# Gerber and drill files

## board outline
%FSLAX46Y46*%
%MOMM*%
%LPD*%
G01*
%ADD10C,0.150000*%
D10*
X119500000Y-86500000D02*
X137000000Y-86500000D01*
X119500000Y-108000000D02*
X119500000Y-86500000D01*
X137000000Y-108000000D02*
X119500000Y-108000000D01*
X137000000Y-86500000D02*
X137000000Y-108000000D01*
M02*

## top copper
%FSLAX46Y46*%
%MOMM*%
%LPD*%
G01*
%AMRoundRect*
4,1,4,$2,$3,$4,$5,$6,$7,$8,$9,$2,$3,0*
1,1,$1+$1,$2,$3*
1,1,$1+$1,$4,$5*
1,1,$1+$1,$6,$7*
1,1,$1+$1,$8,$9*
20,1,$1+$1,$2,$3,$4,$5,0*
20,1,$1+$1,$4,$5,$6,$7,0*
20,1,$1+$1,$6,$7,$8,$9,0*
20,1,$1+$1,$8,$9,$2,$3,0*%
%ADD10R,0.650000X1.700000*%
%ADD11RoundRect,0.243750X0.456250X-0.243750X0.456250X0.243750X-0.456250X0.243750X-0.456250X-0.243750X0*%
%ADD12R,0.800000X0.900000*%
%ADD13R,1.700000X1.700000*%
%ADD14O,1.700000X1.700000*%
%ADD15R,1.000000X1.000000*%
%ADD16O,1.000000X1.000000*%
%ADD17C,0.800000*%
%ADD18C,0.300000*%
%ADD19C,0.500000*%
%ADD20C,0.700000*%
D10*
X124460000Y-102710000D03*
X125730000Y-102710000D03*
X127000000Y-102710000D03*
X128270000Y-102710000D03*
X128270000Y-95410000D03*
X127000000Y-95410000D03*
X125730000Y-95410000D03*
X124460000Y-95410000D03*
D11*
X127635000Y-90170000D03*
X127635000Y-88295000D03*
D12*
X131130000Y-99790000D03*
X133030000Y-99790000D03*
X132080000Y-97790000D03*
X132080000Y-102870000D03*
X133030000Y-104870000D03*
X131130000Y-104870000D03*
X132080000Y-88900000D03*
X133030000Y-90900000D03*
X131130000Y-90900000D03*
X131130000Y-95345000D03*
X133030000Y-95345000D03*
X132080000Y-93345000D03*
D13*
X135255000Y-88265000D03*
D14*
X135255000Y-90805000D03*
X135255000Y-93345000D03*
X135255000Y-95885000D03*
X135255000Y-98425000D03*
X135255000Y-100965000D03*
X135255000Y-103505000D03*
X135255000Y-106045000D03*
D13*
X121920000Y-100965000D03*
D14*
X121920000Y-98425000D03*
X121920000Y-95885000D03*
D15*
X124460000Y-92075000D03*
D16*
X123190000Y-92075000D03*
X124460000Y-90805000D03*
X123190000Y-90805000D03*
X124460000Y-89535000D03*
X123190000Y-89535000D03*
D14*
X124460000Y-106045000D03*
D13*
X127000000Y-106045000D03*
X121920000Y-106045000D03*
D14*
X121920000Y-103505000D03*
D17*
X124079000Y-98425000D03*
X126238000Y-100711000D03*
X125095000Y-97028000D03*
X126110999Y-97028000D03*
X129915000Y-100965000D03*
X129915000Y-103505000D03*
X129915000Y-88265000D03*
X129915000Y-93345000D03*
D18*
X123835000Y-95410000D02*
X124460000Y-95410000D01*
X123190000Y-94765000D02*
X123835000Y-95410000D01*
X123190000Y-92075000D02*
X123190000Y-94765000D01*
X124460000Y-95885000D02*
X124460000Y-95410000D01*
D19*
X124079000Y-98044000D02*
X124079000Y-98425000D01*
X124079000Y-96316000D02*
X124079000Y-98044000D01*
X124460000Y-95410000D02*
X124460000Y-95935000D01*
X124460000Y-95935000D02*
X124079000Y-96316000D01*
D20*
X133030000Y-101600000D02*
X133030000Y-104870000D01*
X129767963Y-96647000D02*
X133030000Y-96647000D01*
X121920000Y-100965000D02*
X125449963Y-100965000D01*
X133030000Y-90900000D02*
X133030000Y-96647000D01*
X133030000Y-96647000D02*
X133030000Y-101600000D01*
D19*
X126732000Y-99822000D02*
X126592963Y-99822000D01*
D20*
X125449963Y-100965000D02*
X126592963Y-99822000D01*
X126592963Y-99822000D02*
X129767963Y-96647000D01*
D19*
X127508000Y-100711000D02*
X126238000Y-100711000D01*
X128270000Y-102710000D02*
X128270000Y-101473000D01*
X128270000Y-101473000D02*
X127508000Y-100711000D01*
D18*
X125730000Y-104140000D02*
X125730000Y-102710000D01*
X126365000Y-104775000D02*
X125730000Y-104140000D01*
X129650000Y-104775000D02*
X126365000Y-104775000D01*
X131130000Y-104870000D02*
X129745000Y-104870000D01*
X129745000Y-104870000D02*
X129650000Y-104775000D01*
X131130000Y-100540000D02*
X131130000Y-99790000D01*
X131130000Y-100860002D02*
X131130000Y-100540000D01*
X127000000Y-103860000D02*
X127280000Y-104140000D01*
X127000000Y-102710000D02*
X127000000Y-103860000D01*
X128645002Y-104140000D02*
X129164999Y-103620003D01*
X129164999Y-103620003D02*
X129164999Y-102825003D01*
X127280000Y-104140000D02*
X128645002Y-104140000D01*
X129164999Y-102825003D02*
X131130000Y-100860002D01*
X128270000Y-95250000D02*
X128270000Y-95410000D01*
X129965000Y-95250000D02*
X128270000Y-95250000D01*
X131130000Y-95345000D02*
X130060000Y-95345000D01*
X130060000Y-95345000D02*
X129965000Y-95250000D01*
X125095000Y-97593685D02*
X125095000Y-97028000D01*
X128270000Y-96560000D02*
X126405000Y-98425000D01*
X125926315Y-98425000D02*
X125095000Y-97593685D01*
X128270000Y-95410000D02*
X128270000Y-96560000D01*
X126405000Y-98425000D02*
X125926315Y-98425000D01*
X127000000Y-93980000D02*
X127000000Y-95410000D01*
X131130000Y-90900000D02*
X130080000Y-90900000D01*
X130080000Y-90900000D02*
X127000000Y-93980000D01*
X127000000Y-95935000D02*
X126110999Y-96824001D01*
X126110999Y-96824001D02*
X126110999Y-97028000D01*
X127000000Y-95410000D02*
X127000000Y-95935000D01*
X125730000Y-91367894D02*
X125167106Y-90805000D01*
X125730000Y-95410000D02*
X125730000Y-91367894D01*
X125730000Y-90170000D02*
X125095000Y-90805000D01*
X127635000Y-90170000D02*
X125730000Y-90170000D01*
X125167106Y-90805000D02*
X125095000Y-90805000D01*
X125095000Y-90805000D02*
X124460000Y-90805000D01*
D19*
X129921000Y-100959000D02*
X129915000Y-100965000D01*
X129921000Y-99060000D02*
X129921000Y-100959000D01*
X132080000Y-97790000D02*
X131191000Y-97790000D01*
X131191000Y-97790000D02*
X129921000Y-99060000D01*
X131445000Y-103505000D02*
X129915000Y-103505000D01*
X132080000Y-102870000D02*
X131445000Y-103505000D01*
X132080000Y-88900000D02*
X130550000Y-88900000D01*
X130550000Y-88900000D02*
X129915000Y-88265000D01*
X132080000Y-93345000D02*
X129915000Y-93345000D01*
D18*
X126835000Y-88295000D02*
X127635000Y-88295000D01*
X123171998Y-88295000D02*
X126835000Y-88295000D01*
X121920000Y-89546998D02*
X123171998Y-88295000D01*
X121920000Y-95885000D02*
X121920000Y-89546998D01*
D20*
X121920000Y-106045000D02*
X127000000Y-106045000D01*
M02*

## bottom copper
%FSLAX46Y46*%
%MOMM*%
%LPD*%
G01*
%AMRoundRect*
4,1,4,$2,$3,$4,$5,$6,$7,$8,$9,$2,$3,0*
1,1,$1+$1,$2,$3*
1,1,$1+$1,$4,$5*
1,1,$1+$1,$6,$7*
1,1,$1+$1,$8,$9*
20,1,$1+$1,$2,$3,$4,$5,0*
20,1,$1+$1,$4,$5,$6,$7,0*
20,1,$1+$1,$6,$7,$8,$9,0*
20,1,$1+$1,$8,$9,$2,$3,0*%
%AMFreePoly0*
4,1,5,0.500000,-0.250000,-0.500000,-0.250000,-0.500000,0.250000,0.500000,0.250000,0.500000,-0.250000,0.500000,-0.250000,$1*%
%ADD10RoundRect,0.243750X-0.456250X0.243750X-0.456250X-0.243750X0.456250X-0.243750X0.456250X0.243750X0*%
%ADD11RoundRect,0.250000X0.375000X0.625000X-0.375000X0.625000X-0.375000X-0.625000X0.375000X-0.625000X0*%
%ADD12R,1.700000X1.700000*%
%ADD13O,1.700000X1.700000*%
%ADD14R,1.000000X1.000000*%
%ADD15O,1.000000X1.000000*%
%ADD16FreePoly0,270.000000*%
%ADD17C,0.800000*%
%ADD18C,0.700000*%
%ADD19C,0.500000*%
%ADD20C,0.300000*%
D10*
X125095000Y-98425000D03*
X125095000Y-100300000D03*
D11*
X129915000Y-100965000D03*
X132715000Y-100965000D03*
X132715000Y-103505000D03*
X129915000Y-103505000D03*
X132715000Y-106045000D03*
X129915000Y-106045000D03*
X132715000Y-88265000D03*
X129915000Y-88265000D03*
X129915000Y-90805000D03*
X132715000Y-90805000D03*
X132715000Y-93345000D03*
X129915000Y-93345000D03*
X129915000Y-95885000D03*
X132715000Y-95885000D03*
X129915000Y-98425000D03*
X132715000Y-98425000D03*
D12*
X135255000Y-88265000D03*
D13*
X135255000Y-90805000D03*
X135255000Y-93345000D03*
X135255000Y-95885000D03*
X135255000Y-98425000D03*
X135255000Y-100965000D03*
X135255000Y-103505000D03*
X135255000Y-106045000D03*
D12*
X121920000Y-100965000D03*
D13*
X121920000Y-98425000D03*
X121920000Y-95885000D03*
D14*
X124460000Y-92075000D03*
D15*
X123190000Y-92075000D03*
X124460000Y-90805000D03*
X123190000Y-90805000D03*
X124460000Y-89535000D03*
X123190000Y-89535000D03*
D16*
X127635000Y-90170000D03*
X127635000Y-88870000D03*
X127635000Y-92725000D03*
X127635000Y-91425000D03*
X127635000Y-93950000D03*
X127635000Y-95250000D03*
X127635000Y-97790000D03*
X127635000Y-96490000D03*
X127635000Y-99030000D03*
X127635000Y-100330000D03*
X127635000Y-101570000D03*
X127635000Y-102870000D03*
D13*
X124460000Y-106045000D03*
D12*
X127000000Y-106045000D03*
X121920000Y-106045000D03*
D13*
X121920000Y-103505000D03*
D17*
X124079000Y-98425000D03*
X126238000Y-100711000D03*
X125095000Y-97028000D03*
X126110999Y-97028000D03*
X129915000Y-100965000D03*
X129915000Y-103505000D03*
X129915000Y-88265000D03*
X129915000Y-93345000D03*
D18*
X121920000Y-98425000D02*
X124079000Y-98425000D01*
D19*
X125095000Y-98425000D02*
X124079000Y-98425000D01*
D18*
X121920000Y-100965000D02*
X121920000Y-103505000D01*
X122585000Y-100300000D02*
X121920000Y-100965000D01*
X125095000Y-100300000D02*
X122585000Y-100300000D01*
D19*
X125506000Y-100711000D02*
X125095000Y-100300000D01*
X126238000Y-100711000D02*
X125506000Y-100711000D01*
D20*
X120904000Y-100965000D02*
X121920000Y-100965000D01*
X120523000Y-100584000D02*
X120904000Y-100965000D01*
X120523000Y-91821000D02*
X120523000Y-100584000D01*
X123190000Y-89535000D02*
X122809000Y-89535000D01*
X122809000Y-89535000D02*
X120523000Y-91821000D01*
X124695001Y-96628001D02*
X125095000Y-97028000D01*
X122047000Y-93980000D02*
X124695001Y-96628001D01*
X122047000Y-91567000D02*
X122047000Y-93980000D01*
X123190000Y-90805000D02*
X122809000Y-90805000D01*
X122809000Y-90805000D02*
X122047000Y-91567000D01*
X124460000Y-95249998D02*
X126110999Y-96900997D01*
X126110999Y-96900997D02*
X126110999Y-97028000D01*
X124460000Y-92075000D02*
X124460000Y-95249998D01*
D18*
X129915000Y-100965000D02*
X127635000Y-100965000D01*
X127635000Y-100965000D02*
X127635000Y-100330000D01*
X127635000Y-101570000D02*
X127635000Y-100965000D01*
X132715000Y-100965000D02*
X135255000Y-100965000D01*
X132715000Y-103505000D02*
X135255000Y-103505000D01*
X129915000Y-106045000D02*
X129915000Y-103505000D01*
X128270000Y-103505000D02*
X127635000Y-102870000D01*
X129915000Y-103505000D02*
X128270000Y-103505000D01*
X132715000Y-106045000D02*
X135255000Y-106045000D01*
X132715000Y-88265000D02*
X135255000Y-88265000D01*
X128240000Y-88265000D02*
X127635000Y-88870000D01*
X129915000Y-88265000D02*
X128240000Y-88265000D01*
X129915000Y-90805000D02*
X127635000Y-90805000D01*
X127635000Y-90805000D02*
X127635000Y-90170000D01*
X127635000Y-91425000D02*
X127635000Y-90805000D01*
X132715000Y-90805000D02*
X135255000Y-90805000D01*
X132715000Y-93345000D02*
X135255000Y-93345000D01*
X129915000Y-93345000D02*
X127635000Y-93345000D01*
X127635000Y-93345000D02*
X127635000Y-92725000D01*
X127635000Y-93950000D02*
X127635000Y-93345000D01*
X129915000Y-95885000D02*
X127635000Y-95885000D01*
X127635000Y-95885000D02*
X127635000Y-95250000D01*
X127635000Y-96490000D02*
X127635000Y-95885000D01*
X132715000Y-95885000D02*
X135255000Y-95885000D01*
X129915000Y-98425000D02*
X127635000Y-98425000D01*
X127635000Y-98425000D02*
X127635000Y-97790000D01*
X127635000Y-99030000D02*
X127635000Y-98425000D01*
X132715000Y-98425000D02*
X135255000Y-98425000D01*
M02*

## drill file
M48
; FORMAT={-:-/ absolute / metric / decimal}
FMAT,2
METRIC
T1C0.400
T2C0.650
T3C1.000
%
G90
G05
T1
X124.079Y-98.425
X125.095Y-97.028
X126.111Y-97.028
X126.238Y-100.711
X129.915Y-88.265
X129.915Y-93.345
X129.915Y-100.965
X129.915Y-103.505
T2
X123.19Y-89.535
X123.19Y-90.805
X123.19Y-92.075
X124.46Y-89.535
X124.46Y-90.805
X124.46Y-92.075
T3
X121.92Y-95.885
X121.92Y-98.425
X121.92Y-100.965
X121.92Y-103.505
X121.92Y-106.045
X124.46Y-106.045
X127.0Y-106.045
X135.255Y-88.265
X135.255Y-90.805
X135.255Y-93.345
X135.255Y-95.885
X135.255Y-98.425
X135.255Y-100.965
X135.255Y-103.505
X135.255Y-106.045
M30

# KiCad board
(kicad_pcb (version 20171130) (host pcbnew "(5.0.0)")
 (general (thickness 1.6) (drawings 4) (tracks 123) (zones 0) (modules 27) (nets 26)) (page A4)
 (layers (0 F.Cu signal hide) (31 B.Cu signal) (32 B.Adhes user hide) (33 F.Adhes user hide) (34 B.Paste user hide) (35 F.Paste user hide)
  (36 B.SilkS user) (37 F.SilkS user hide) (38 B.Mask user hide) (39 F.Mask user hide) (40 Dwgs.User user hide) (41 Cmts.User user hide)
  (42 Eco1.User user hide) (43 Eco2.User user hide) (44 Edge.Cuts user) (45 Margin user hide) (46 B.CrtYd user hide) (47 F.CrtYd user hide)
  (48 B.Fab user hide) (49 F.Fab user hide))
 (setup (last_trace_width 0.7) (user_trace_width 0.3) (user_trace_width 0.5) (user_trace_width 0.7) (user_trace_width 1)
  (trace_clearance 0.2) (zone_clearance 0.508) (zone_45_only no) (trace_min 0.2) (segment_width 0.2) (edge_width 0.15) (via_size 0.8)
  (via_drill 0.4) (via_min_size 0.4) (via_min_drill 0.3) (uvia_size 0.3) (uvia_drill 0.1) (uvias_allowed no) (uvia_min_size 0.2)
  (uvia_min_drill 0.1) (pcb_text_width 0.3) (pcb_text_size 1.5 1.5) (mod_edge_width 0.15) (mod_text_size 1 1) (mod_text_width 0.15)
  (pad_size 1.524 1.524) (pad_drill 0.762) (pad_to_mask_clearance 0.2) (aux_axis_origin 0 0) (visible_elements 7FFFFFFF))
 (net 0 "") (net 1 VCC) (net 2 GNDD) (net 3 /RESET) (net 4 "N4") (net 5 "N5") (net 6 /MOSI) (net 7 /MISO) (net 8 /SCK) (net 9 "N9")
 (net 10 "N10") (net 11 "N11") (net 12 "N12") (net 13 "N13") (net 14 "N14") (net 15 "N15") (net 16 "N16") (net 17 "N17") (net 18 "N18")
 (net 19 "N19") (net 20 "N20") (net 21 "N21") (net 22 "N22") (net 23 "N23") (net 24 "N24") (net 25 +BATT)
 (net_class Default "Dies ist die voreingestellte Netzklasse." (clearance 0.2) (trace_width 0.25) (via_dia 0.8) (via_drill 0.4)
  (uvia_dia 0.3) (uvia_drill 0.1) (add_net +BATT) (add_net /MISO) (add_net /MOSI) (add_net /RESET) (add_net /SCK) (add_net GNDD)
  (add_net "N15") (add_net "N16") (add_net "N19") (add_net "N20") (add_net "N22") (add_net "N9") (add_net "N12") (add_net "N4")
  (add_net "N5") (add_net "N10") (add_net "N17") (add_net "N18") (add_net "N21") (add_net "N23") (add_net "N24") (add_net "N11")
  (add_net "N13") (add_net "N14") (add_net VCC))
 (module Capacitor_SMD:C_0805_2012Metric (layer B.Cu) (at 125.095 99.3625 270)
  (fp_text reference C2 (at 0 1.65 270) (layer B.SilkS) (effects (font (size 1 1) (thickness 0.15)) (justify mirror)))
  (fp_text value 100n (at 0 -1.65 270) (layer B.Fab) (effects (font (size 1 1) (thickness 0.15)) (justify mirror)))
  (pad 1 smd roundrect (at -0.9375 0 270) (size 0.975 1.4) (layers B.Cu B.Paste B.Mask) (roundrect_rratio 0.25) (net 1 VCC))
  (pad 2 smd roundrect (at 0.9375 0 270) (size 0.975 1.4) (layers B.Cu B.Paste B.Mask) (roundrect_rratio 0.25) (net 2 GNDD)))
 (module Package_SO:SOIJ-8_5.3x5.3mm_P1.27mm (layer F.Cu) (at 126.365 99.06 90)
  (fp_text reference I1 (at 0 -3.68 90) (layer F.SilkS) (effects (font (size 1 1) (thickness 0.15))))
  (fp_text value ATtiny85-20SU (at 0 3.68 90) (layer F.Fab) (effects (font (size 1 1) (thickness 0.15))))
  (pad 1 smd rect (at -3.65 -1.905 90) (size 1.7 0.65) (layers F.Cu F.Paste F.Mask) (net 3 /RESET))
  (pad 2 smd rect (at -3.65 -0.635 90) (size 1.7 0.65) (layers F.Cu F.Paste F.Mask) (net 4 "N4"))
  (pad 3 smd rect (at -3.65 0.635 90) (size 1.7 0.65) (layers F.Cu F.Paste F.Mask) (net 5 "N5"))
  (pad 4 smd rect (at -3.65 1.905 90) (size 1.7 0.65) (layers F.Cu F.Paste F.Mask) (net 2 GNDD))
  (pad 5 smd rect (at 3.65 1.905 90) (size 1.7 0.65) (layers F.Cu F.Paste F.Mask) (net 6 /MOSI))
  (pad 6 smd rect (at 3.65 0.635 90) (size 1.7 0.65) (layers F.Cu F.Paste F.Mask) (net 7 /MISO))
  (pad 7 smd rect (at 3.65 -0.635 90) (size 1.7 0.65) (layers F.Cu F.Paste F.Mask) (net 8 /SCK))
  (pad 8 smd rect (at 3.65 -1.905 90) (size 1.7 0.65) (layers F.Cu F.Paste F.Mask) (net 1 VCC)))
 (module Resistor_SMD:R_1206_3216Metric (layer B.Cu) (at 131.315 100.965 180)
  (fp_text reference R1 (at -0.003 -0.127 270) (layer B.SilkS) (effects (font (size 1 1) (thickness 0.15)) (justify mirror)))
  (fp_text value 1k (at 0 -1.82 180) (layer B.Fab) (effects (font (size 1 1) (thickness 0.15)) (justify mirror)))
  (pad 2 smd roundrect (at 1.4 0 180) (size 1.25 1.75) (layers B.Cu B.Paste B.Mask) (roundrect_rratio 0.2) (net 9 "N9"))
  (pad 1 smd roundrect (at -1.4 0 180) (size 1.25 1.75) (layers B.Cu B.Paste B.Mask) (roundrect_rratio 0.2) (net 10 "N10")))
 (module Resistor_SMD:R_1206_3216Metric (layer B.Cu) (at 131.315 103.505 180)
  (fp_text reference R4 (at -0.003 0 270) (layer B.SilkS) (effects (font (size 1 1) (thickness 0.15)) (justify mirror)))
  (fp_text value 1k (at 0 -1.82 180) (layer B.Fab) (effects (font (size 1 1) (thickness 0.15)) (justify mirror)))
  (pad 1 smd roundrect (at -1.4 0 180) (size 1.25 1.75) (layers B.Cu B.Paste B.Mask) (roundrect_rratio 0.2) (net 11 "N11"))
  (pad 2 smd roundrect (at 1.4 0 180) (size 1.25 1.75) (layers B.Cu B.Paste B.Mask) (roundrect_rratio 0.2) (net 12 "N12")))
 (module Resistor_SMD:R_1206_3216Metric (layer B.Cu) (at 131.315 106.045 180)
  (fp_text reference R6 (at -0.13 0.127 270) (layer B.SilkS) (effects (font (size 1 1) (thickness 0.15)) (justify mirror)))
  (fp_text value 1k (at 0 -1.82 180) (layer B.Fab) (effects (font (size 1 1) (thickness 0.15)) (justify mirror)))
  (pad 1 smd roundrect (at -1.4 0 180) (size 1.25 1.75) (layers B.Cu B.Paste B.Mask) (roundrect_rratio 0.2) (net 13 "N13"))
  (pad 2 smd roundrect (at 1.4 0 180) (size 1.25 1.75) (layers B.Cu B.Paste B.Mask) (roundrect_rratio 0.2) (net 12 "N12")))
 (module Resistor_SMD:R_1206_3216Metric (layer B.Cu) (at 131.315 88.265 180)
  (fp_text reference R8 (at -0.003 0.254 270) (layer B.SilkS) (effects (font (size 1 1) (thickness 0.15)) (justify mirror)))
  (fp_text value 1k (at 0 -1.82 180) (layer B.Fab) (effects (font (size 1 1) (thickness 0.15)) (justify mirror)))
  (pad 1 smd roundrect (at -1.4 0 180) (size 1.25 1.75) (layers B.Cu B.Paste B.Mask) (roundrect_rratio 0.2) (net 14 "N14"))
  (pad 2 smd roundrect (at 1.4 0 180) (size 1.25 1.75) (layers B.Cu B.Paste B.Mask) (roundrect_rratio 0.2) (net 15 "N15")))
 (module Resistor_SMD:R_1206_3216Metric (layer B.Cu) (at 131.315 90.805 180)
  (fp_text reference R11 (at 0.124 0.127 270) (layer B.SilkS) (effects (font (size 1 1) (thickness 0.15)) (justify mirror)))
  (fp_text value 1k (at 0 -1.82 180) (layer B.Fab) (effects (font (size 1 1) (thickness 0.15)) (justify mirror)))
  (pad 2 smd roundrect (at 1.4 0 180) (size 1.25 1.75) (layers B.Cu B.Paste B.Mask) (roundrect_rratio 0.2) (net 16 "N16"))
  (pad 1 smd roundrect (at -1.4 0 180) (size 1.25 1.75) (layers B.Cu B.Paste B.Mask) (roundrect_rratio 0.2) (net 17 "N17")))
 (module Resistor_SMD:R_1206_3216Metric (layer B.Cu) (at 131.315 93.345 180)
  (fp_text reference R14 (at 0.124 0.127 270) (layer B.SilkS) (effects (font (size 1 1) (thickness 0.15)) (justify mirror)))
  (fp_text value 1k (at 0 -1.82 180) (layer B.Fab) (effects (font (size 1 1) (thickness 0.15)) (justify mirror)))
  (pad 1 smd roundrect (at -1.4 0 180) (size 1.25 1.75) (layers B.Cu B.Paste B.Mask) (roundrect_rratio 0.2) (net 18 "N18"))
  (pad 2 smd roundrect (at 1.4 0 180) (size 1.25 1.75) (layers B.Cu B.Paste B.Mask) (roundrect_rratio 0.2) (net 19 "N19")))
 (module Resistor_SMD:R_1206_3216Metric (layer B.Cu) (at 131.315 95.885 180)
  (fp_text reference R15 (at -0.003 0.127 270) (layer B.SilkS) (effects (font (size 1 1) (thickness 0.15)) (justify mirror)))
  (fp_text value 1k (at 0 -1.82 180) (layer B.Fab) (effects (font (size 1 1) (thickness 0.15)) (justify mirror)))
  (pad 2 smd roundrect (at 1.4 0 180) (size 1.25 1.75) (layers B.Cu B.Paste B.Mask) (roundrect_rratio 0.2) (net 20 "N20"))
  (pad 1 smd roundrect (at -1.4 0 180) (size 1.25 1.75) (layers B.Cu B.Paste B.Mask) (roundrect_rratio 0.2) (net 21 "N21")))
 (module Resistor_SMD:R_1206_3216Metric (layer B.Cu) (at 131.315 98.425 180)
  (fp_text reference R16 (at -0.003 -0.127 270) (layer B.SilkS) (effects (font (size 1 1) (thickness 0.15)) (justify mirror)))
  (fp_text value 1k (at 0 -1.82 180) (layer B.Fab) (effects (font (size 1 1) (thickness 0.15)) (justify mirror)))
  (pad 2 smd roundrect (at 1.4 0 180) (size 1.25 1.75) (layers B.Cu B.Paste B.Mask) (roundrect_rratio 0.2) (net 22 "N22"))
  (pad 1 smd roundrect (at -1.4 0 180) (size 1.25 1.75) (layers B.Cu B.Paste B.Mask) (roundrect_rratio 0.2) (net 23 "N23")))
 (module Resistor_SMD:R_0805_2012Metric (layer F.Cu) (at 127.635 89.2325 90)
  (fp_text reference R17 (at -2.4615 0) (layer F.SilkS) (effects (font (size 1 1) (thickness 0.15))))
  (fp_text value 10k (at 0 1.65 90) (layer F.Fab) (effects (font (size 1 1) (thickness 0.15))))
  (pad 1 smd roundrect (at -0.9375 0 90) (size 0.975 1.4) (layers F.Cu F.Paste F.Mask) (roundrect_rratio 0.25) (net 8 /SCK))
  (pad 2 smd roundrect (at 0.9375 0 90) (size 0.975 1.4) (layers F.Cu F.Paste F.Mask) (roundrect_rratio 0.25) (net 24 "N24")))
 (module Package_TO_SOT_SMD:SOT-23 (layer F.Cu) (at 132.08 98.79 90)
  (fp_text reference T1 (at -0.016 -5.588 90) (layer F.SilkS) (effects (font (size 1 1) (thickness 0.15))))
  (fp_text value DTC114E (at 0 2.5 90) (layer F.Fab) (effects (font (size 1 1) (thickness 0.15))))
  (pad 1 smd rect (at -1 -0.95 90) (size 0.9 0.8) (layers F.Cu F.Paste F.Mask) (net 5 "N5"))
  (pad 2 smd rect (at -1 0.95 90) (size 0.9 0.8) (layers F.Cu F.Paste F.Mask) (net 2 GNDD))
  (pad 3 smd rect (at 1 0 90) (size 0.9 0.8) (layers F.Cu F.Paste F.Mask) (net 9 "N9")))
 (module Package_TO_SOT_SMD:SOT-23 (layer F.Cu) (at 132.08 103.87 90)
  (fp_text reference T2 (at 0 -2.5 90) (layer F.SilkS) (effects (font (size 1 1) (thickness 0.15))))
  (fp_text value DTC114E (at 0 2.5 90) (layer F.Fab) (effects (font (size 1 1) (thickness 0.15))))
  (pad 3 smd rect (at 1 0 90) (size 0.9 0.8) (layers F.Cu F.Paste F.Mask) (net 12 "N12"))
  (pad 2 smd rect (at -1 0.95 90) (size 0.9 0.8) (layers F.Cu F.Paste F.Mask) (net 2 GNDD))
  (pad 1 smd rect (at -1 -0.95 90) (size 0.9 0.8) (layers F.Cu F.Paste F.Mask) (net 4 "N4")))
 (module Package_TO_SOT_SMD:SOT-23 (layer F.Cu) (at 132.08 89.9 90)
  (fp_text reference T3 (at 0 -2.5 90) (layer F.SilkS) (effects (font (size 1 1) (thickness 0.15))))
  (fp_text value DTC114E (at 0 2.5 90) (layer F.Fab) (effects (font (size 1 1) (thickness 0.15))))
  (pad 3 smd rect (at 1 0 90) (size 0.9 0.8) (layers F.Cu F.Paste F.Mask) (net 15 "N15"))
  (pad 2 smd rect (at -1 0.95 90) (size 0.9 0.8) (layers F.Cu F.Paste F.Mask) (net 2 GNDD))
  (pad 1 smd rect (at -1 -0.95 90) (size 0.9 0.8) (layers F.Cu F.Paste F.Mask) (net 7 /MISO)))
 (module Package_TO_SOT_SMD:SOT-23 (layer F.Cu) (at 132.08 94.345 90)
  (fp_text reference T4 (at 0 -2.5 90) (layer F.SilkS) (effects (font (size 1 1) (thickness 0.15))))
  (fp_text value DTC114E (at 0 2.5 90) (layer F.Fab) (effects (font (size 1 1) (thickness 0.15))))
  (pad 1 smd rect (at -1 -0.95 90) (size 0.9 0.8) (layers F.Cu F.Paste F.Mask) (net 6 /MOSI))
  (pad 2 smd rect (at -1 0.95 90) (size 0.9 0.8) (layers F.Cu F.Paste F.Mask) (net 2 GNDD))
  (pad 3 smd rect (at 1 0 90) (size 0.9 0.8) (layers F.Cu F.Paste F.Mask) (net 19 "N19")))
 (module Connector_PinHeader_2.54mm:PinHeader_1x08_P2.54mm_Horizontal (layer F.Cu) (at 135.255 88.265)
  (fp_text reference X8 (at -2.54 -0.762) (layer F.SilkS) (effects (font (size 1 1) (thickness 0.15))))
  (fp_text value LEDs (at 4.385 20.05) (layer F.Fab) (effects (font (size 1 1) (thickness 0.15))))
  (pad 1 thru_hole rect (at 0 0) (size 1.7 1.7) (drill 1) (layers *.Cu *.Mask) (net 14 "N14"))
  (pad 2 thru_hole oval (at 0 2.54) (size 1.7 1.7) (drill 1) (layers *.Cu *.Mask) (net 17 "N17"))
  (pad 3 thru_hole oval (at 0 5.08) (size 1.7 1.7) (drill 1) (layers *.Cu *.Mask) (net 18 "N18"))
  (pad 4 thru_hole oval (at 0 7.62) (size 1.7 1.7) (drill 1) (layers *.Cu *.Mask) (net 21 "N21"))
  (pad 5 thru_hole oval (at 0 10.16) (size 1.7 1.7) (drill 1) (layers *.Cu *.Mask) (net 23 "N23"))
  (pad 6 thru_hole oval (at 0 12.7) (size 1.7 1.7) (drill 1) (layers *.Cu *.Mask) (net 10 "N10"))
  (pad 7 thru_hole oval (at 0 15.24) (size 1.7 1.7) (drill 1) (layers *.Cu *.Mask) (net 11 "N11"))
  (pad 8 thru_hole oval (at 0 17.78) (size 1.7 1.7) (drill 1) (layers *.Cu *.Mask) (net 13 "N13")))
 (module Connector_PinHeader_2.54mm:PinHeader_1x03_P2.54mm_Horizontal (layer F.Cu) (at 121.92 100.965 180)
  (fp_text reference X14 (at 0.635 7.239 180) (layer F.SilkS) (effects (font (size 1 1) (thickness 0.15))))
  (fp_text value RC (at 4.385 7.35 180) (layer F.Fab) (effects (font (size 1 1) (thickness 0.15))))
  (pad 1 thru_hole rect (at 0 0 180) (size 1.7 1.7) (drill 1) (layers *.Cu *.Mask) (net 2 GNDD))
  (pad 2 thru_hole oval (at 0 2.54 180) (size 1.7 1.7) (drill 1) (layers *.Cu *.Mask) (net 1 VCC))
  (pad 3 thru_hole oval (at 0 5.08 180) (size 1.7 1.7) (drill 1) (layers *.Cu *.Mask) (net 24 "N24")))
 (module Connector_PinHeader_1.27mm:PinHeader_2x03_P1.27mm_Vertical (layer F.Cu) (at 124.46 92.075 180)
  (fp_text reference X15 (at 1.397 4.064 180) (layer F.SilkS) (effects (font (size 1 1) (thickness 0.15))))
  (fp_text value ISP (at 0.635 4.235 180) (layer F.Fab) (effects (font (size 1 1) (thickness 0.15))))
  (pad 1 thru_hole rect (at 0 0 180) (size 1 1) (drill 0.65) (layers *.Cu *.Mask) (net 7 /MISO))
  (pad 2 thru_hole oval (at 1.27 0 180) (size 1 1) (drill 0.65) (layers *.Cu *.Mask) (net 1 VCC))
  (pad 3 thru_hole oval (at 0 1.27 180) (size 1 1) (drill 0.65) (layers *.Cu *.Mask) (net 8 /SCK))
  (pad 4 thru_hole oval (at 1.27 1.27 180) (size 1 1) (drill 0.65) (layers *.Cu *.Mask) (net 6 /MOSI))
  (pad 5 thru_hole oval (at 0 2.54 180) (size 1 1) (drill 0.65) (layers *.Cu *.Mask) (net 3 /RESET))
  (pad 6 thru_hole oval (at 1.27 2.54 180) (size 1 1) (drill 0.65) (layers *.Cu *.Mask) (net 2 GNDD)))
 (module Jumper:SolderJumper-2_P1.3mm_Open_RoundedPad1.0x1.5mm (layer B.Cu) (at 127.635 89.52 270)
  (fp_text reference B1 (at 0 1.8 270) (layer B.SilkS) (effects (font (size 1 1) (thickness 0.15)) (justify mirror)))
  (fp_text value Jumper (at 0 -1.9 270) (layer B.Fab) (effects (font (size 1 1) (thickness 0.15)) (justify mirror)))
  (pad 2 smd custom (at 0.65 0 270) (size 1 0.5) (layers B.Cu B.Mask) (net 16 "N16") (zone_connect 0)
   (options (clearance outline) (anchor rect)) (primitives))
  (pad 1 smd custom (at -0.65 0 270) (size 1 0.5) (layers B.Cu B.Mask) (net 15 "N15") (zone_connect 0)
   (options (clearance outline) (anchor rect)) (primitives)))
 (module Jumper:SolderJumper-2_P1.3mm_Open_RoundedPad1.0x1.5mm (layer B.Cu) (at 127.635 92.075 270)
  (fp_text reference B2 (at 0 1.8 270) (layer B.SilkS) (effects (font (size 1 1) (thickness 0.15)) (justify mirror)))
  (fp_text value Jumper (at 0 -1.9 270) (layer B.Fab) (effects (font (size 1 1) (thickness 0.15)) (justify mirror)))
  (pad 2 smd custom (at 0.65 0 270) (size 1 0.5) (layers B.Cu B.Mask) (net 19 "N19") (zone_connect 0)
   (options (clearance outline) (anchor rect)) (primitives))
  (pad 1 smd custom (at -0.65 0 270) (size 1 0.5) (layers B.Cu B.Mask) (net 16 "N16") (zone_connect 0)
   (options (clearance outline) (anchor rect)) (primitives)))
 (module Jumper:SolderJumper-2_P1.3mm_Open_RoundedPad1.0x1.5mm (layer B.Cu) (at 127.635 94.6 270)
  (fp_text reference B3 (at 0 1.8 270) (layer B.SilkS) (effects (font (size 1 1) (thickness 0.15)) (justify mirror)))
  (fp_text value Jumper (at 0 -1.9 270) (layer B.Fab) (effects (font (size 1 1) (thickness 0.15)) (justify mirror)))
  (pad 1 smd custom (at -0.65 0 270) (size 1 0.5) (layers B.Cu B.Mask) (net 19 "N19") (zone_connect 0)
   (options (clearance outline) (anchor rect)) (primitives))
  (pad 2 smd custom (at 0.65 0 270) (size 1 0.5) (layers B.Cu B.Mask) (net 20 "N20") (zone_connect 0)
   (options (clearance outline) (anchor rect)) (primitives)))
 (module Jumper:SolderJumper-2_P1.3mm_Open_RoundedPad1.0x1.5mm (layer B.Cu) (at 127.635 97.14 270)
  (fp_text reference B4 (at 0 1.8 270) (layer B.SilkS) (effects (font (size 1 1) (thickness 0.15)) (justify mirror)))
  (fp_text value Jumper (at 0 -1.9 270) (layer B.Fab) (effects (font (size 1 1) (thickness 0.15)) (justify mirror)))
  (pad 2 smd custom (at 0.65 0 270) (size 1 0.5) (layers B.Cu B.Mask) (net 22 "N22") (zone_connect 0)
   (options (clearance outline) (anchor rect)) (primitives))
  (pad 1 smd custom (at -0.65 0 270) (size 1 0.5) (layers B.Cu B.Mask) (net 20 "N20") (zone_connect 0)
   (options (clearance outline) (anchor rect)) (primitives)))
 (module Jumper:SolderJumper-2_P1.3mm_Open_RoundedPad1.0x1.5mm (layer B.Cu) (at 127.635 99.68 270)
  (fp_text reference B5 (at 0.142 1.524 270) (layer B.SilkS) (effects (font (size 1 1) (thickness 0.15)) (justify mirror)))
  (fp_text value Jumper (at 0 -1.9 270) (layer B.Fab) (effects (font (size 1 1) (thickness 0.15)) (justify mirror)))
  (pad 1 smd custom (at -0.65 0 270) (size 1 0.5) (layers B.Cu B.Mask) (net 22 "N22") (zone_connect 0)
   (options (clearance outline) (anchor rect)) (primitives))
  (pad 2 smd custom (at 0.65 0 270) (size 1 0.5) (layers B.Cu B.Mask) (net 9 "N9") (zone_connect 0)
   (options (clearance outline) (anchor rect)) (primitives)))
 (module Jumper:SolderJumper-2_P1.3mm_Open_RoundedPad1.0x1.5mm (layer B.Cu) (at 127.635 102.22 270)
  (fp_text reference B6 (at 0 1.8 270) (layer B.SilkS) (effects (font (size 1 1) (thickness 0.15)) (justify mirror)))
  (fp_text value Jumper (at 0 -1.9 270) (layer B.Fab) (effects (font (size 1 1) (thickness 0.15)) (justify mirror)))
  (pad 1 smd custom (at -0.65 0 270) (size 1 0.5) (layers B.Cu B.Mask) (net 9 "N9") (zone_connect 0)
   (options (clearance outline) (anchor rect)) (primitives))
  (pad 2 smd custom (at 0.65 0 270) (size 1 0.5) (layers B.Cu B.Mask) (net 12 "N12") (zone_connect 0)
   (options (clearance outline) (anchor rect)) (primitives)))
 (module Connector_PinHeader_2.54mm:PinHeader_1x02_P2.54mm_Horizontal (layer F.Cu) (at 127 106.045 270)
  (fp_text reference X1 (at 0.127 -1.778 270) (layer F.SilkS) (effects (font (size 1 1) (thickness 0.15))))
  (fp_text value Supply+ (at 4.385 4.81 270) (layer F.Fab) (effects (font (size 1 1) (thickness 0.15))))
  (pad 2 thru_hole oval (at 0 2.54 270) (size 1.7 1.7) (drill 1) (layers *.Cu *.Mask) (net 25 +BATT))
  (pad 1 thru_hole rect (at 0 0 270) (size 1.7 1.7) (drill 1) (layers *.Cu *.Mask) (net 25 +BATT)))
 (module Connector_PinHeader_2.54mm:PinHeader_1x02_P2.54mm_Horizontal (layer F.Cu) (at 121.92 106.045 180)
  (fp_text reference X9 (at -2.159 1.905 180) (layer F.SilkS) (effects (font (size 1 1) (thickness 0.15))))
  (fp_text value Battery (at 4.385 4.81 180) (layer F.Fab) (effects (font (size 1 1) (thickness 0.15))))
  (pad 1 thru_hole rect (at 0 0 180) (size 1.7 1.7) (drill 1) (layers *.Cu *.Mask) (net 25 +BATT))
  (pad 2 thru_hole oval (at 0 2.54 180) (size 1.7 1.7) (drill 1) (layers *.Cu *.Mask) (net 2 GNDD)))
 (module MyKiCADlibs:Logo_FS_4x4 (layer B.Cu) (at 123.825 90.805 180)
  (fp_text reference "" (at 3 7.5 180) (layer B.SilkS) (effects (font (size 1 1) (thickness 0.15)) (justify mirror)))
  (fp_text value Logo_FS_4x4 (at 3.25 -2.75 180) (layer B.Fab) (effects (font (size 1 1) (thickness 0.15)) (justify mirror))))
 (gr_line (start 119.5 86.5) (end 137 86.5) (layer Edge.Cuts) (width 0.15))
 (gr_line (start 119.5 108) (end 119.5 86.5) (layer Edge.Cuts) (width 0.15))
 (gr_line (start 137 108) (end 119.5 108) (layer Edge.Cuts) (width 0.15))
 (gr_line (start 137 86.5) (end 137 108) (layer Edge.Cuts) (width 0.15))
 (segment (start 123.835 95.41) (end 124.46 95.41) (width 0.3) (layer F.Cu) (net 1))
 (segment (start 123.19 94.765) (end 123.835 95.41) (width 0.3) (layer F.Cu) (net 1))
 (segment (start 123.19 92.075) (end 123.19 94.765) (width 0.3) (layer F.Cu) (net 1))
 (segment (start 124.46 95.885) (end 124.46 95.41) (width 0.3) (layer F.Cu) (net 1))
 (segment (start 121.92 98.425) (end 124.079 98.425) (width 0.7) (layer B.Cu) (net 1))
 (segment (start 125.095 98.425) (end 124.079 98.425) (width 0.5) (layer B.Cu) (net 1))
 (via (at 124.079 98.425) (size 0.8) (drill 0.4) (layers F.Cu B.Cu) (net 1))
 (segment (start 124.079 98.044) (end 124.079 98.425) (width 0.5) (layer F.Cu) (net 1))
 (segment (start 124.079 96.316) (end 124.079 98.044) (width 0.5) (layer F.Cu) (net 1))
 (segment (start 124.46 95.41) (end 124.46 95.935) (width 0.5) (layer F.Cu) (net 1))
 (segment (start 124.46 95.935) (end 124.079 96.316) (width 0.5) (layer F.Cu) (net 1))
 (segment (start 133.03 101.6) (end 133.03 104.87) (width 0.7) (layer F.Cu) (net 2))
 (segment (start 121.92 100.965) (end 121.92 103.505) (width 0.7) (layer B.Cu) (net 2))
 (segment (start 122.585 100.3) (end 121.92 100.965) (width 0.7) (layer B.Cu) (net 2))
 (segment (start 125.095 100.3) (end 122.585 100.3) (width 0.7) (layer B.Cu) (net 2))
 (segment (start 129.767963 96.647) (end 133.03 96.647) (width 0.7) (layer F.Cu) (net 2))
 (segment (start 121.92 100.965) (end 125.449963 100.965) (width 0.7) (layer F.Cu) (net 2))
 (segment (start 133.03 90.9) (end 133.03 96.647) (width 0.7) (layer F.Cu) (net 2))
 (segment (start 133.03 96.647) (end 133.03 101.6) (width 0.7) (layer F.Cu) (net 2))
 (segment (start 126.732 99.822) (end 126.592963 99.822) (width 0.5) (layer F.Cu) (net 2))
 (segment (start 125.449963 100.965) (end 126.592963 99.822) (width 0.7) (layer F.Cu) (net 2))
 (segment (start 126.592963 99.822) (end 129.767963 96.647) (width 0.7) (layer F.Cu) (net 2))
 (via (at 126.238 100.711) (size 0.8) (drill 0.4) (layers F.Cu B.Cu) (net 2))
 (segment (start 125.506 100.711) (end 125.095 100.3) (width 0.5) (layer B.Cu) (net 2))
 (segment (start 126.238 100.711) (end 125.506 100.711) (width 0.5) (layer B.Cu) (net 2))
 (segment (start 127.508 100.711) (end 126.238 100.711) (width 0.5) (layer F.Cu) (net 2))
 (segment (start 128.27 102.71) (end 128.27 101.473) (width 0.5) (layer F.Cu) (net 2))
 (segment (start 128.27 101.473) (end 127.508 100.711) (width 0.5) (layer F.Cu) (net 2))
 (segment (start 120.904 100.965) (end 121.92 100.965) (width 0.3) (layer B.Cu) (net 2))
 (segment (start 120.523 100.584) (end 120.904 100.965) (width 0.3) (layer B.Cu) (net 2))
 (segment (start 120.523 91.821) (end 120.523 100.584) (width 0.3) (layer B.Cu) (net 2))
 (segment (start 123.19 89.535) (end 122.809 89.535) (width 0.3) (layer B.Cu) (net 2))
 (segment (start 122.809 89.535) (end 120.523 91.821) (width 0.3) (layer B.Cu) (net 2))
 (segment (start 125.73 104.14) (end 125.73 102.71) (width 0.3) (layer F.Cu) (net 4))
 (segment (start 126.365 104.775) (end 125.73 104.14) (width 0.3) (layer F.Cu) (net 4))
 (segment (start 129.65 104.775) (end 126.365 104.775) (width 0.3) (layer F.Cu) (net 4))
 (segment (start 131.13 104.87) (end 129.745 104.87) (width 0.3) (layer F.Cu) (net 4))
 (segment (start 129.745 104.87) (end 129.65 104.775) (width 0.3) (layer F.Cu) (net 4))
 (segment (start 131.13 100.54) (end 131.13 99.79) (width 0.3) (layer F.Cu) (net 5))
 (segment (start 131.13 100.860002) (end 131.13 100.54) (width 0.3) (layer F.Cu) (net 5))
 (segment (start 127 103.86) (end 127.28 104.14) (width 0.3) (layer F.Cu) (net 5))
 (segment (start 127 102.71) (end 127 103.86) (width 0.3) (layer F.Cu) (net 5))
 (segment (start 128.645002 104.14) (end 129.164999 103.620003) (width 0.3) (layer F.Cu) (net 5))
 (segment (start 129.164999 103.620003) (end 129.164999 102.825003) (width 0.3) (layer F.Cu) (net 5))
 (segment (start 127.28 104.14) (end 128.645002 104.14) (width 0.3) (layer F.Cu) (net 5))
 (segment (start 129.164999 102.825003) (end 131.13 100.860002) (width 0.3) (layer F.Cu) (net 5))
 (segment (start 128.27 95.25) (end 128.27 95.41) (width 0.3) (layer F.Cu) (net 6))
 (segment (start 129.965 95.25) (end 128.27 95.25) (width 0.3) (layer F.Cu) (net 6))
 (segment (start 131.13 95.345) (end 130.06 95.345) (width 0.3) (layer F.Cu) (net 6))
 (segment (start 130.06 95.345) (end 129.965 95.25) (width 0.3) (layer F.Cu) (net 6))
 (via (at 125.095 97.028) (size 0.8) (drill 0.4) (layers F.Cu B.Cu) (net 6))
 (segment (start 125.095 97.593685) (end 125.095 97.028) (width 0.3) (layer F.Cu) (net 6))
 (segment (start 128.27 96.56) (end 126.405 98.425) (width 0.3) (layer F.Cu) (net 6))
 (segment (start 125.926315 98.425) (end 125.095 97.593685) (width 0.3) (layer F.Cu) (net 6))
 (segment (start 128.27 95.41) (end 128.27 96.56) (width 0.3) (layer F.Cu) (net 6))
 (segment (start 126.405 98.425) (end 125.926315 98.425) (width 0.3) (layer F.Cu) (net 6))
 (segment (start 124.695001 96.628001) (end 125.095 97.028) (width 0.3) (layer B.Cu) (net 6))
 (segment (start 122.047 93.98) (end 124.695001 96.628001) (width 0.3) (layer B.Cu) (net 6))
 (segment (start 122.047 91.567) (end 122.047 93.98) (width 0.3) (layer B.Cu) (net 6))
 (segment (start 123.19 90.805) (end 122.809 90.805) (width 0.3) (layer B.Cu) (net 6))
 (segment (start 122.809 90.805) (end 122.047 91.567) (width 0.3) (layer B.Cu) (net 6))
 (segment (start 127 93.98) (end 127 95.41) (width 0.3) (layer F.Cu) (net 7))
 (segment (start 131.13 90.9) (end 130.08 90.9) (width 0.3) (layer F.Cu) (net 7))
 (segment (start 130.08 90.9) (end 127 93.98) (width 0.3) (layer F.Cu) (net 7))
 (via (at 126.110999 97.028) (size 0.8) (drill 0.4) (layers F.Cu B.Cu) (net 7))
 (segment (start 124.46 95.249998) (end 126.110999 96.900997) (width 0.3) (layer B.Cu) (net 7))
 (segment (start 126.110999 96.900997) (end 126.110999 97.028) (width 0.3) (layer B.Cu) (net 7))
 (segment (start 127 95.935) (end 126.110999 96.824001) (width 0.3) (layer F.Cu) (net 7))
 (segment (start 124.46 92.075) (end 124.46 95.249998) (width 0.3) (layer B.Cu) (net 7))
 (segment (start 126.110999 96.824001) (end 126.110999 97.028) (width 0.3) (layer F.Cu) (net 7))
 (segment (start 127 95.41) (end 127 95.935) (width 0.3) (layer F.Cu) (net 7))
 (segment (start 125.73 91.367894) (end 125.167106 90.805) (width 0.3) (layer F.Cu) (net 8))
 (segment (start 125.73 95.41) (end 125.73 91.367894) (width 0.3) (layer F.Cu) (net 8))
 (segment (start 125.73 90.17) (end 125.095 90.805) (width 0.3) (layer F.Cu) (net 8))
 (segment (start 127.635 90.17) (end 125.73 90.17) (width 0.3) (layer F.Cu) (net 8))
 (segment (start 125.167106 90.805) (end 125.095 90.805) (width 0.3) (layer F.Cu) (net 8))
 (segment (start 125.095 90.805) (end 124.46 90.805) (width 0.3) (layer F.Cu) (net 8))
 (segment (start 129.915 100.965) (end 127.635 100.965) (width 0.7) (layer B.Cu) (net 9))
 (segment (start 127.635 100.965) (end 127.635 100.33) (width 0.7) (layer B.Cu) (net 9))
 (segment (start 127.635 101.57) (end 127.635 100.965) (width 0.7) (layer B.Cu) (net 9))
 (via (at 129.915 100.965) (size 0.8) (drill 0.4) (layers F.Cu B.Cu) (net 9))
 (segment (start 129.921 100.959) (end 129.915 100.965) (width 0.5) (layer F.Cu) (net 9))
 (segment (start 129.921 99.06) (end 129.921 100.959) (width 0.5) (layer F.Cu) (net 9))
 (segment (start 132.08 97.79) (end 131.191 97.79) (width 0.5) (layer F.Cu) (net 9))
 (segment (start 131.191 97.79) (end 129.921 99.06) (width 0.5) (layer F.Cu) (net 9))
 (segment (start 132.715 100.965) (end 135.255 100.965) (width 0.7) (layer B.Cu) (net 10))
 (segment (start 132.715 103.505) (end 135.255 103.505) (width 0.7) (layer B.Cu) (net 11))
 (segment (start 129.915 106.045) (end 129.915 103.505) (width 0.7) (layer B.Cu) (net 12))
 (segment (start 128.27 103.505) (end 127.635 102.87) (width 0.7) (layer B.Cu) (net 12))
 (segment (start 129.915 103.505) (end 128.27 103.505) (width 0.7) (layer B.Cu) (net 12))
 (via (at 129.915 103.505) (size 0.8) (drill 0.4) (layers F.Cu B.Cu) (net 12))
 (segment (start 131.445 103.505) (end 129.915 103.505) (width 0.5) (layer F.Cu) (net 12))
 (segment (start 132.08 102.87) (end 131.445 103.505) (width 0.5) (layer F.Cu) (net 12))
 (segment (start 132.715 106.045) (end 135.255 106.045) (width 0.7) (layer B.Cu) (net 13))
 (segment (start 132.715 88.265) (end 135.255 88.265) (width 0.7) (layer B.Cu) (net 14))
 (segment (start 128.24 88.265) (end 127.635 88.87) (width 0.7) (layer B.Cu) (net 15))
 (segment (start 129.915 88.265) (end 128.24 88.265) (width 0.7) (layer B.Cu) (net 15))
 (via (at 129.915 88.265) (size 0.8) (drill 0.4) (layers F.Cu B.Cu) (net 15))
 (segment (start 132.08 88.9) (end 130.55 88.9) (width 0.5) (layer F.Cu) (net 15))
 (segment (start 130.55 88.9) (end 129.915 88.265) (width 0.5) (layer F.Cu) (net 15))
 (segment (start 129.915 90.805) (end 127.635 90.805) (width 0.7) (layer B.Cu) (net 16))
 (segment (start 127.635 90.805) (end 127.635 90.17) (width 0.7) (layer B.Cu) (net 16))
 (segment (start 127.635 91.425) (end 127.635 90.805) (width 0.7) (layer B.Cu) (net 16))
 (segment (start 132.715 90.805) (end 135.255 90.805) (width 0.7) (layer B.Cu) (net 17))
 (segment (start 132.715 93.345) (end 135.255 93.345) (width 0.7) (layer B.Cu) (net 18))
 (segment (start 129.915 93.345) (end 127.635 93.345) (width 0.7) (layer B.Cu) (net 19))
 (segment (start 127.635 93.345) (end 127.635 92.725) (width 0.7) (layer B.Cu) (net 19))
 (segment (start 127.635 93.95) (end 127.635 93.345) (width 0.7) (layer B.Cu) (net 19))
 (via (at 129.915 93.345) (size 0.8) (drill 0.4) (layers F.Cu B.Cu) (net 19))
 (segment (start 132.08 93.345) (end 129.915 93.345) (width 0.5) (layer F.Cu) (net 19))
 (segment (start 129.915 95.885) (end 127.635 95.885) (width 0.7) (layer B.Cu) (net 20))
 (segment (start 127.635 95.885) (end 127.635 95.25) (width 0.7) (layer B.Cu) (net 20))
 (segment (start 127.635 96.49) (end 127.635 95.885) (width 0.7) (layer B.Cu) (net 20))
 (segment (start 132.715 95.885) (end 135.255 95.885) (width 0.7) (layer B.Cu) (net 21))
 (segment (start 129.915 98.425) (end 127.635 98.425) (width 0.7) (layer B.Cu) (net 22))
 (segment (start 127.635 98.425) (end 127.635 97.79) (width 0.7) (layer B.Cu) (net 22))
 (segment (start 127.635 99.03) (end 127.635 98.425) (width 0.7) (layer B.Cu) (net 22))
 (segment (start 132.715 98.425) (end 135.255 98.425) (width 0.7) (layer B.Cu) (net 23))
 (segment (start 126.835 88.295) (end 127.635 88.295) (width 0.3) (layer F.Cu) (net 24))
 (segment (start 123.171998 88.295) (end 126.835 88.295) (width 0.3) (layer F.Cu) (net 24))
 (segment (start 121.92 89.546998) (end 123.171998 88.295) (width 0.3) (layer F.Cu) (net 24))
 (segment (start 121.92 95.885) (end 121.92 89.546998) (width 0.3) (layer F.Cu) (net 24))
 (segment (start 121.92 106.045) (end 127 106.045) (width 0.7) (layer F.Cu) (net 25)))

